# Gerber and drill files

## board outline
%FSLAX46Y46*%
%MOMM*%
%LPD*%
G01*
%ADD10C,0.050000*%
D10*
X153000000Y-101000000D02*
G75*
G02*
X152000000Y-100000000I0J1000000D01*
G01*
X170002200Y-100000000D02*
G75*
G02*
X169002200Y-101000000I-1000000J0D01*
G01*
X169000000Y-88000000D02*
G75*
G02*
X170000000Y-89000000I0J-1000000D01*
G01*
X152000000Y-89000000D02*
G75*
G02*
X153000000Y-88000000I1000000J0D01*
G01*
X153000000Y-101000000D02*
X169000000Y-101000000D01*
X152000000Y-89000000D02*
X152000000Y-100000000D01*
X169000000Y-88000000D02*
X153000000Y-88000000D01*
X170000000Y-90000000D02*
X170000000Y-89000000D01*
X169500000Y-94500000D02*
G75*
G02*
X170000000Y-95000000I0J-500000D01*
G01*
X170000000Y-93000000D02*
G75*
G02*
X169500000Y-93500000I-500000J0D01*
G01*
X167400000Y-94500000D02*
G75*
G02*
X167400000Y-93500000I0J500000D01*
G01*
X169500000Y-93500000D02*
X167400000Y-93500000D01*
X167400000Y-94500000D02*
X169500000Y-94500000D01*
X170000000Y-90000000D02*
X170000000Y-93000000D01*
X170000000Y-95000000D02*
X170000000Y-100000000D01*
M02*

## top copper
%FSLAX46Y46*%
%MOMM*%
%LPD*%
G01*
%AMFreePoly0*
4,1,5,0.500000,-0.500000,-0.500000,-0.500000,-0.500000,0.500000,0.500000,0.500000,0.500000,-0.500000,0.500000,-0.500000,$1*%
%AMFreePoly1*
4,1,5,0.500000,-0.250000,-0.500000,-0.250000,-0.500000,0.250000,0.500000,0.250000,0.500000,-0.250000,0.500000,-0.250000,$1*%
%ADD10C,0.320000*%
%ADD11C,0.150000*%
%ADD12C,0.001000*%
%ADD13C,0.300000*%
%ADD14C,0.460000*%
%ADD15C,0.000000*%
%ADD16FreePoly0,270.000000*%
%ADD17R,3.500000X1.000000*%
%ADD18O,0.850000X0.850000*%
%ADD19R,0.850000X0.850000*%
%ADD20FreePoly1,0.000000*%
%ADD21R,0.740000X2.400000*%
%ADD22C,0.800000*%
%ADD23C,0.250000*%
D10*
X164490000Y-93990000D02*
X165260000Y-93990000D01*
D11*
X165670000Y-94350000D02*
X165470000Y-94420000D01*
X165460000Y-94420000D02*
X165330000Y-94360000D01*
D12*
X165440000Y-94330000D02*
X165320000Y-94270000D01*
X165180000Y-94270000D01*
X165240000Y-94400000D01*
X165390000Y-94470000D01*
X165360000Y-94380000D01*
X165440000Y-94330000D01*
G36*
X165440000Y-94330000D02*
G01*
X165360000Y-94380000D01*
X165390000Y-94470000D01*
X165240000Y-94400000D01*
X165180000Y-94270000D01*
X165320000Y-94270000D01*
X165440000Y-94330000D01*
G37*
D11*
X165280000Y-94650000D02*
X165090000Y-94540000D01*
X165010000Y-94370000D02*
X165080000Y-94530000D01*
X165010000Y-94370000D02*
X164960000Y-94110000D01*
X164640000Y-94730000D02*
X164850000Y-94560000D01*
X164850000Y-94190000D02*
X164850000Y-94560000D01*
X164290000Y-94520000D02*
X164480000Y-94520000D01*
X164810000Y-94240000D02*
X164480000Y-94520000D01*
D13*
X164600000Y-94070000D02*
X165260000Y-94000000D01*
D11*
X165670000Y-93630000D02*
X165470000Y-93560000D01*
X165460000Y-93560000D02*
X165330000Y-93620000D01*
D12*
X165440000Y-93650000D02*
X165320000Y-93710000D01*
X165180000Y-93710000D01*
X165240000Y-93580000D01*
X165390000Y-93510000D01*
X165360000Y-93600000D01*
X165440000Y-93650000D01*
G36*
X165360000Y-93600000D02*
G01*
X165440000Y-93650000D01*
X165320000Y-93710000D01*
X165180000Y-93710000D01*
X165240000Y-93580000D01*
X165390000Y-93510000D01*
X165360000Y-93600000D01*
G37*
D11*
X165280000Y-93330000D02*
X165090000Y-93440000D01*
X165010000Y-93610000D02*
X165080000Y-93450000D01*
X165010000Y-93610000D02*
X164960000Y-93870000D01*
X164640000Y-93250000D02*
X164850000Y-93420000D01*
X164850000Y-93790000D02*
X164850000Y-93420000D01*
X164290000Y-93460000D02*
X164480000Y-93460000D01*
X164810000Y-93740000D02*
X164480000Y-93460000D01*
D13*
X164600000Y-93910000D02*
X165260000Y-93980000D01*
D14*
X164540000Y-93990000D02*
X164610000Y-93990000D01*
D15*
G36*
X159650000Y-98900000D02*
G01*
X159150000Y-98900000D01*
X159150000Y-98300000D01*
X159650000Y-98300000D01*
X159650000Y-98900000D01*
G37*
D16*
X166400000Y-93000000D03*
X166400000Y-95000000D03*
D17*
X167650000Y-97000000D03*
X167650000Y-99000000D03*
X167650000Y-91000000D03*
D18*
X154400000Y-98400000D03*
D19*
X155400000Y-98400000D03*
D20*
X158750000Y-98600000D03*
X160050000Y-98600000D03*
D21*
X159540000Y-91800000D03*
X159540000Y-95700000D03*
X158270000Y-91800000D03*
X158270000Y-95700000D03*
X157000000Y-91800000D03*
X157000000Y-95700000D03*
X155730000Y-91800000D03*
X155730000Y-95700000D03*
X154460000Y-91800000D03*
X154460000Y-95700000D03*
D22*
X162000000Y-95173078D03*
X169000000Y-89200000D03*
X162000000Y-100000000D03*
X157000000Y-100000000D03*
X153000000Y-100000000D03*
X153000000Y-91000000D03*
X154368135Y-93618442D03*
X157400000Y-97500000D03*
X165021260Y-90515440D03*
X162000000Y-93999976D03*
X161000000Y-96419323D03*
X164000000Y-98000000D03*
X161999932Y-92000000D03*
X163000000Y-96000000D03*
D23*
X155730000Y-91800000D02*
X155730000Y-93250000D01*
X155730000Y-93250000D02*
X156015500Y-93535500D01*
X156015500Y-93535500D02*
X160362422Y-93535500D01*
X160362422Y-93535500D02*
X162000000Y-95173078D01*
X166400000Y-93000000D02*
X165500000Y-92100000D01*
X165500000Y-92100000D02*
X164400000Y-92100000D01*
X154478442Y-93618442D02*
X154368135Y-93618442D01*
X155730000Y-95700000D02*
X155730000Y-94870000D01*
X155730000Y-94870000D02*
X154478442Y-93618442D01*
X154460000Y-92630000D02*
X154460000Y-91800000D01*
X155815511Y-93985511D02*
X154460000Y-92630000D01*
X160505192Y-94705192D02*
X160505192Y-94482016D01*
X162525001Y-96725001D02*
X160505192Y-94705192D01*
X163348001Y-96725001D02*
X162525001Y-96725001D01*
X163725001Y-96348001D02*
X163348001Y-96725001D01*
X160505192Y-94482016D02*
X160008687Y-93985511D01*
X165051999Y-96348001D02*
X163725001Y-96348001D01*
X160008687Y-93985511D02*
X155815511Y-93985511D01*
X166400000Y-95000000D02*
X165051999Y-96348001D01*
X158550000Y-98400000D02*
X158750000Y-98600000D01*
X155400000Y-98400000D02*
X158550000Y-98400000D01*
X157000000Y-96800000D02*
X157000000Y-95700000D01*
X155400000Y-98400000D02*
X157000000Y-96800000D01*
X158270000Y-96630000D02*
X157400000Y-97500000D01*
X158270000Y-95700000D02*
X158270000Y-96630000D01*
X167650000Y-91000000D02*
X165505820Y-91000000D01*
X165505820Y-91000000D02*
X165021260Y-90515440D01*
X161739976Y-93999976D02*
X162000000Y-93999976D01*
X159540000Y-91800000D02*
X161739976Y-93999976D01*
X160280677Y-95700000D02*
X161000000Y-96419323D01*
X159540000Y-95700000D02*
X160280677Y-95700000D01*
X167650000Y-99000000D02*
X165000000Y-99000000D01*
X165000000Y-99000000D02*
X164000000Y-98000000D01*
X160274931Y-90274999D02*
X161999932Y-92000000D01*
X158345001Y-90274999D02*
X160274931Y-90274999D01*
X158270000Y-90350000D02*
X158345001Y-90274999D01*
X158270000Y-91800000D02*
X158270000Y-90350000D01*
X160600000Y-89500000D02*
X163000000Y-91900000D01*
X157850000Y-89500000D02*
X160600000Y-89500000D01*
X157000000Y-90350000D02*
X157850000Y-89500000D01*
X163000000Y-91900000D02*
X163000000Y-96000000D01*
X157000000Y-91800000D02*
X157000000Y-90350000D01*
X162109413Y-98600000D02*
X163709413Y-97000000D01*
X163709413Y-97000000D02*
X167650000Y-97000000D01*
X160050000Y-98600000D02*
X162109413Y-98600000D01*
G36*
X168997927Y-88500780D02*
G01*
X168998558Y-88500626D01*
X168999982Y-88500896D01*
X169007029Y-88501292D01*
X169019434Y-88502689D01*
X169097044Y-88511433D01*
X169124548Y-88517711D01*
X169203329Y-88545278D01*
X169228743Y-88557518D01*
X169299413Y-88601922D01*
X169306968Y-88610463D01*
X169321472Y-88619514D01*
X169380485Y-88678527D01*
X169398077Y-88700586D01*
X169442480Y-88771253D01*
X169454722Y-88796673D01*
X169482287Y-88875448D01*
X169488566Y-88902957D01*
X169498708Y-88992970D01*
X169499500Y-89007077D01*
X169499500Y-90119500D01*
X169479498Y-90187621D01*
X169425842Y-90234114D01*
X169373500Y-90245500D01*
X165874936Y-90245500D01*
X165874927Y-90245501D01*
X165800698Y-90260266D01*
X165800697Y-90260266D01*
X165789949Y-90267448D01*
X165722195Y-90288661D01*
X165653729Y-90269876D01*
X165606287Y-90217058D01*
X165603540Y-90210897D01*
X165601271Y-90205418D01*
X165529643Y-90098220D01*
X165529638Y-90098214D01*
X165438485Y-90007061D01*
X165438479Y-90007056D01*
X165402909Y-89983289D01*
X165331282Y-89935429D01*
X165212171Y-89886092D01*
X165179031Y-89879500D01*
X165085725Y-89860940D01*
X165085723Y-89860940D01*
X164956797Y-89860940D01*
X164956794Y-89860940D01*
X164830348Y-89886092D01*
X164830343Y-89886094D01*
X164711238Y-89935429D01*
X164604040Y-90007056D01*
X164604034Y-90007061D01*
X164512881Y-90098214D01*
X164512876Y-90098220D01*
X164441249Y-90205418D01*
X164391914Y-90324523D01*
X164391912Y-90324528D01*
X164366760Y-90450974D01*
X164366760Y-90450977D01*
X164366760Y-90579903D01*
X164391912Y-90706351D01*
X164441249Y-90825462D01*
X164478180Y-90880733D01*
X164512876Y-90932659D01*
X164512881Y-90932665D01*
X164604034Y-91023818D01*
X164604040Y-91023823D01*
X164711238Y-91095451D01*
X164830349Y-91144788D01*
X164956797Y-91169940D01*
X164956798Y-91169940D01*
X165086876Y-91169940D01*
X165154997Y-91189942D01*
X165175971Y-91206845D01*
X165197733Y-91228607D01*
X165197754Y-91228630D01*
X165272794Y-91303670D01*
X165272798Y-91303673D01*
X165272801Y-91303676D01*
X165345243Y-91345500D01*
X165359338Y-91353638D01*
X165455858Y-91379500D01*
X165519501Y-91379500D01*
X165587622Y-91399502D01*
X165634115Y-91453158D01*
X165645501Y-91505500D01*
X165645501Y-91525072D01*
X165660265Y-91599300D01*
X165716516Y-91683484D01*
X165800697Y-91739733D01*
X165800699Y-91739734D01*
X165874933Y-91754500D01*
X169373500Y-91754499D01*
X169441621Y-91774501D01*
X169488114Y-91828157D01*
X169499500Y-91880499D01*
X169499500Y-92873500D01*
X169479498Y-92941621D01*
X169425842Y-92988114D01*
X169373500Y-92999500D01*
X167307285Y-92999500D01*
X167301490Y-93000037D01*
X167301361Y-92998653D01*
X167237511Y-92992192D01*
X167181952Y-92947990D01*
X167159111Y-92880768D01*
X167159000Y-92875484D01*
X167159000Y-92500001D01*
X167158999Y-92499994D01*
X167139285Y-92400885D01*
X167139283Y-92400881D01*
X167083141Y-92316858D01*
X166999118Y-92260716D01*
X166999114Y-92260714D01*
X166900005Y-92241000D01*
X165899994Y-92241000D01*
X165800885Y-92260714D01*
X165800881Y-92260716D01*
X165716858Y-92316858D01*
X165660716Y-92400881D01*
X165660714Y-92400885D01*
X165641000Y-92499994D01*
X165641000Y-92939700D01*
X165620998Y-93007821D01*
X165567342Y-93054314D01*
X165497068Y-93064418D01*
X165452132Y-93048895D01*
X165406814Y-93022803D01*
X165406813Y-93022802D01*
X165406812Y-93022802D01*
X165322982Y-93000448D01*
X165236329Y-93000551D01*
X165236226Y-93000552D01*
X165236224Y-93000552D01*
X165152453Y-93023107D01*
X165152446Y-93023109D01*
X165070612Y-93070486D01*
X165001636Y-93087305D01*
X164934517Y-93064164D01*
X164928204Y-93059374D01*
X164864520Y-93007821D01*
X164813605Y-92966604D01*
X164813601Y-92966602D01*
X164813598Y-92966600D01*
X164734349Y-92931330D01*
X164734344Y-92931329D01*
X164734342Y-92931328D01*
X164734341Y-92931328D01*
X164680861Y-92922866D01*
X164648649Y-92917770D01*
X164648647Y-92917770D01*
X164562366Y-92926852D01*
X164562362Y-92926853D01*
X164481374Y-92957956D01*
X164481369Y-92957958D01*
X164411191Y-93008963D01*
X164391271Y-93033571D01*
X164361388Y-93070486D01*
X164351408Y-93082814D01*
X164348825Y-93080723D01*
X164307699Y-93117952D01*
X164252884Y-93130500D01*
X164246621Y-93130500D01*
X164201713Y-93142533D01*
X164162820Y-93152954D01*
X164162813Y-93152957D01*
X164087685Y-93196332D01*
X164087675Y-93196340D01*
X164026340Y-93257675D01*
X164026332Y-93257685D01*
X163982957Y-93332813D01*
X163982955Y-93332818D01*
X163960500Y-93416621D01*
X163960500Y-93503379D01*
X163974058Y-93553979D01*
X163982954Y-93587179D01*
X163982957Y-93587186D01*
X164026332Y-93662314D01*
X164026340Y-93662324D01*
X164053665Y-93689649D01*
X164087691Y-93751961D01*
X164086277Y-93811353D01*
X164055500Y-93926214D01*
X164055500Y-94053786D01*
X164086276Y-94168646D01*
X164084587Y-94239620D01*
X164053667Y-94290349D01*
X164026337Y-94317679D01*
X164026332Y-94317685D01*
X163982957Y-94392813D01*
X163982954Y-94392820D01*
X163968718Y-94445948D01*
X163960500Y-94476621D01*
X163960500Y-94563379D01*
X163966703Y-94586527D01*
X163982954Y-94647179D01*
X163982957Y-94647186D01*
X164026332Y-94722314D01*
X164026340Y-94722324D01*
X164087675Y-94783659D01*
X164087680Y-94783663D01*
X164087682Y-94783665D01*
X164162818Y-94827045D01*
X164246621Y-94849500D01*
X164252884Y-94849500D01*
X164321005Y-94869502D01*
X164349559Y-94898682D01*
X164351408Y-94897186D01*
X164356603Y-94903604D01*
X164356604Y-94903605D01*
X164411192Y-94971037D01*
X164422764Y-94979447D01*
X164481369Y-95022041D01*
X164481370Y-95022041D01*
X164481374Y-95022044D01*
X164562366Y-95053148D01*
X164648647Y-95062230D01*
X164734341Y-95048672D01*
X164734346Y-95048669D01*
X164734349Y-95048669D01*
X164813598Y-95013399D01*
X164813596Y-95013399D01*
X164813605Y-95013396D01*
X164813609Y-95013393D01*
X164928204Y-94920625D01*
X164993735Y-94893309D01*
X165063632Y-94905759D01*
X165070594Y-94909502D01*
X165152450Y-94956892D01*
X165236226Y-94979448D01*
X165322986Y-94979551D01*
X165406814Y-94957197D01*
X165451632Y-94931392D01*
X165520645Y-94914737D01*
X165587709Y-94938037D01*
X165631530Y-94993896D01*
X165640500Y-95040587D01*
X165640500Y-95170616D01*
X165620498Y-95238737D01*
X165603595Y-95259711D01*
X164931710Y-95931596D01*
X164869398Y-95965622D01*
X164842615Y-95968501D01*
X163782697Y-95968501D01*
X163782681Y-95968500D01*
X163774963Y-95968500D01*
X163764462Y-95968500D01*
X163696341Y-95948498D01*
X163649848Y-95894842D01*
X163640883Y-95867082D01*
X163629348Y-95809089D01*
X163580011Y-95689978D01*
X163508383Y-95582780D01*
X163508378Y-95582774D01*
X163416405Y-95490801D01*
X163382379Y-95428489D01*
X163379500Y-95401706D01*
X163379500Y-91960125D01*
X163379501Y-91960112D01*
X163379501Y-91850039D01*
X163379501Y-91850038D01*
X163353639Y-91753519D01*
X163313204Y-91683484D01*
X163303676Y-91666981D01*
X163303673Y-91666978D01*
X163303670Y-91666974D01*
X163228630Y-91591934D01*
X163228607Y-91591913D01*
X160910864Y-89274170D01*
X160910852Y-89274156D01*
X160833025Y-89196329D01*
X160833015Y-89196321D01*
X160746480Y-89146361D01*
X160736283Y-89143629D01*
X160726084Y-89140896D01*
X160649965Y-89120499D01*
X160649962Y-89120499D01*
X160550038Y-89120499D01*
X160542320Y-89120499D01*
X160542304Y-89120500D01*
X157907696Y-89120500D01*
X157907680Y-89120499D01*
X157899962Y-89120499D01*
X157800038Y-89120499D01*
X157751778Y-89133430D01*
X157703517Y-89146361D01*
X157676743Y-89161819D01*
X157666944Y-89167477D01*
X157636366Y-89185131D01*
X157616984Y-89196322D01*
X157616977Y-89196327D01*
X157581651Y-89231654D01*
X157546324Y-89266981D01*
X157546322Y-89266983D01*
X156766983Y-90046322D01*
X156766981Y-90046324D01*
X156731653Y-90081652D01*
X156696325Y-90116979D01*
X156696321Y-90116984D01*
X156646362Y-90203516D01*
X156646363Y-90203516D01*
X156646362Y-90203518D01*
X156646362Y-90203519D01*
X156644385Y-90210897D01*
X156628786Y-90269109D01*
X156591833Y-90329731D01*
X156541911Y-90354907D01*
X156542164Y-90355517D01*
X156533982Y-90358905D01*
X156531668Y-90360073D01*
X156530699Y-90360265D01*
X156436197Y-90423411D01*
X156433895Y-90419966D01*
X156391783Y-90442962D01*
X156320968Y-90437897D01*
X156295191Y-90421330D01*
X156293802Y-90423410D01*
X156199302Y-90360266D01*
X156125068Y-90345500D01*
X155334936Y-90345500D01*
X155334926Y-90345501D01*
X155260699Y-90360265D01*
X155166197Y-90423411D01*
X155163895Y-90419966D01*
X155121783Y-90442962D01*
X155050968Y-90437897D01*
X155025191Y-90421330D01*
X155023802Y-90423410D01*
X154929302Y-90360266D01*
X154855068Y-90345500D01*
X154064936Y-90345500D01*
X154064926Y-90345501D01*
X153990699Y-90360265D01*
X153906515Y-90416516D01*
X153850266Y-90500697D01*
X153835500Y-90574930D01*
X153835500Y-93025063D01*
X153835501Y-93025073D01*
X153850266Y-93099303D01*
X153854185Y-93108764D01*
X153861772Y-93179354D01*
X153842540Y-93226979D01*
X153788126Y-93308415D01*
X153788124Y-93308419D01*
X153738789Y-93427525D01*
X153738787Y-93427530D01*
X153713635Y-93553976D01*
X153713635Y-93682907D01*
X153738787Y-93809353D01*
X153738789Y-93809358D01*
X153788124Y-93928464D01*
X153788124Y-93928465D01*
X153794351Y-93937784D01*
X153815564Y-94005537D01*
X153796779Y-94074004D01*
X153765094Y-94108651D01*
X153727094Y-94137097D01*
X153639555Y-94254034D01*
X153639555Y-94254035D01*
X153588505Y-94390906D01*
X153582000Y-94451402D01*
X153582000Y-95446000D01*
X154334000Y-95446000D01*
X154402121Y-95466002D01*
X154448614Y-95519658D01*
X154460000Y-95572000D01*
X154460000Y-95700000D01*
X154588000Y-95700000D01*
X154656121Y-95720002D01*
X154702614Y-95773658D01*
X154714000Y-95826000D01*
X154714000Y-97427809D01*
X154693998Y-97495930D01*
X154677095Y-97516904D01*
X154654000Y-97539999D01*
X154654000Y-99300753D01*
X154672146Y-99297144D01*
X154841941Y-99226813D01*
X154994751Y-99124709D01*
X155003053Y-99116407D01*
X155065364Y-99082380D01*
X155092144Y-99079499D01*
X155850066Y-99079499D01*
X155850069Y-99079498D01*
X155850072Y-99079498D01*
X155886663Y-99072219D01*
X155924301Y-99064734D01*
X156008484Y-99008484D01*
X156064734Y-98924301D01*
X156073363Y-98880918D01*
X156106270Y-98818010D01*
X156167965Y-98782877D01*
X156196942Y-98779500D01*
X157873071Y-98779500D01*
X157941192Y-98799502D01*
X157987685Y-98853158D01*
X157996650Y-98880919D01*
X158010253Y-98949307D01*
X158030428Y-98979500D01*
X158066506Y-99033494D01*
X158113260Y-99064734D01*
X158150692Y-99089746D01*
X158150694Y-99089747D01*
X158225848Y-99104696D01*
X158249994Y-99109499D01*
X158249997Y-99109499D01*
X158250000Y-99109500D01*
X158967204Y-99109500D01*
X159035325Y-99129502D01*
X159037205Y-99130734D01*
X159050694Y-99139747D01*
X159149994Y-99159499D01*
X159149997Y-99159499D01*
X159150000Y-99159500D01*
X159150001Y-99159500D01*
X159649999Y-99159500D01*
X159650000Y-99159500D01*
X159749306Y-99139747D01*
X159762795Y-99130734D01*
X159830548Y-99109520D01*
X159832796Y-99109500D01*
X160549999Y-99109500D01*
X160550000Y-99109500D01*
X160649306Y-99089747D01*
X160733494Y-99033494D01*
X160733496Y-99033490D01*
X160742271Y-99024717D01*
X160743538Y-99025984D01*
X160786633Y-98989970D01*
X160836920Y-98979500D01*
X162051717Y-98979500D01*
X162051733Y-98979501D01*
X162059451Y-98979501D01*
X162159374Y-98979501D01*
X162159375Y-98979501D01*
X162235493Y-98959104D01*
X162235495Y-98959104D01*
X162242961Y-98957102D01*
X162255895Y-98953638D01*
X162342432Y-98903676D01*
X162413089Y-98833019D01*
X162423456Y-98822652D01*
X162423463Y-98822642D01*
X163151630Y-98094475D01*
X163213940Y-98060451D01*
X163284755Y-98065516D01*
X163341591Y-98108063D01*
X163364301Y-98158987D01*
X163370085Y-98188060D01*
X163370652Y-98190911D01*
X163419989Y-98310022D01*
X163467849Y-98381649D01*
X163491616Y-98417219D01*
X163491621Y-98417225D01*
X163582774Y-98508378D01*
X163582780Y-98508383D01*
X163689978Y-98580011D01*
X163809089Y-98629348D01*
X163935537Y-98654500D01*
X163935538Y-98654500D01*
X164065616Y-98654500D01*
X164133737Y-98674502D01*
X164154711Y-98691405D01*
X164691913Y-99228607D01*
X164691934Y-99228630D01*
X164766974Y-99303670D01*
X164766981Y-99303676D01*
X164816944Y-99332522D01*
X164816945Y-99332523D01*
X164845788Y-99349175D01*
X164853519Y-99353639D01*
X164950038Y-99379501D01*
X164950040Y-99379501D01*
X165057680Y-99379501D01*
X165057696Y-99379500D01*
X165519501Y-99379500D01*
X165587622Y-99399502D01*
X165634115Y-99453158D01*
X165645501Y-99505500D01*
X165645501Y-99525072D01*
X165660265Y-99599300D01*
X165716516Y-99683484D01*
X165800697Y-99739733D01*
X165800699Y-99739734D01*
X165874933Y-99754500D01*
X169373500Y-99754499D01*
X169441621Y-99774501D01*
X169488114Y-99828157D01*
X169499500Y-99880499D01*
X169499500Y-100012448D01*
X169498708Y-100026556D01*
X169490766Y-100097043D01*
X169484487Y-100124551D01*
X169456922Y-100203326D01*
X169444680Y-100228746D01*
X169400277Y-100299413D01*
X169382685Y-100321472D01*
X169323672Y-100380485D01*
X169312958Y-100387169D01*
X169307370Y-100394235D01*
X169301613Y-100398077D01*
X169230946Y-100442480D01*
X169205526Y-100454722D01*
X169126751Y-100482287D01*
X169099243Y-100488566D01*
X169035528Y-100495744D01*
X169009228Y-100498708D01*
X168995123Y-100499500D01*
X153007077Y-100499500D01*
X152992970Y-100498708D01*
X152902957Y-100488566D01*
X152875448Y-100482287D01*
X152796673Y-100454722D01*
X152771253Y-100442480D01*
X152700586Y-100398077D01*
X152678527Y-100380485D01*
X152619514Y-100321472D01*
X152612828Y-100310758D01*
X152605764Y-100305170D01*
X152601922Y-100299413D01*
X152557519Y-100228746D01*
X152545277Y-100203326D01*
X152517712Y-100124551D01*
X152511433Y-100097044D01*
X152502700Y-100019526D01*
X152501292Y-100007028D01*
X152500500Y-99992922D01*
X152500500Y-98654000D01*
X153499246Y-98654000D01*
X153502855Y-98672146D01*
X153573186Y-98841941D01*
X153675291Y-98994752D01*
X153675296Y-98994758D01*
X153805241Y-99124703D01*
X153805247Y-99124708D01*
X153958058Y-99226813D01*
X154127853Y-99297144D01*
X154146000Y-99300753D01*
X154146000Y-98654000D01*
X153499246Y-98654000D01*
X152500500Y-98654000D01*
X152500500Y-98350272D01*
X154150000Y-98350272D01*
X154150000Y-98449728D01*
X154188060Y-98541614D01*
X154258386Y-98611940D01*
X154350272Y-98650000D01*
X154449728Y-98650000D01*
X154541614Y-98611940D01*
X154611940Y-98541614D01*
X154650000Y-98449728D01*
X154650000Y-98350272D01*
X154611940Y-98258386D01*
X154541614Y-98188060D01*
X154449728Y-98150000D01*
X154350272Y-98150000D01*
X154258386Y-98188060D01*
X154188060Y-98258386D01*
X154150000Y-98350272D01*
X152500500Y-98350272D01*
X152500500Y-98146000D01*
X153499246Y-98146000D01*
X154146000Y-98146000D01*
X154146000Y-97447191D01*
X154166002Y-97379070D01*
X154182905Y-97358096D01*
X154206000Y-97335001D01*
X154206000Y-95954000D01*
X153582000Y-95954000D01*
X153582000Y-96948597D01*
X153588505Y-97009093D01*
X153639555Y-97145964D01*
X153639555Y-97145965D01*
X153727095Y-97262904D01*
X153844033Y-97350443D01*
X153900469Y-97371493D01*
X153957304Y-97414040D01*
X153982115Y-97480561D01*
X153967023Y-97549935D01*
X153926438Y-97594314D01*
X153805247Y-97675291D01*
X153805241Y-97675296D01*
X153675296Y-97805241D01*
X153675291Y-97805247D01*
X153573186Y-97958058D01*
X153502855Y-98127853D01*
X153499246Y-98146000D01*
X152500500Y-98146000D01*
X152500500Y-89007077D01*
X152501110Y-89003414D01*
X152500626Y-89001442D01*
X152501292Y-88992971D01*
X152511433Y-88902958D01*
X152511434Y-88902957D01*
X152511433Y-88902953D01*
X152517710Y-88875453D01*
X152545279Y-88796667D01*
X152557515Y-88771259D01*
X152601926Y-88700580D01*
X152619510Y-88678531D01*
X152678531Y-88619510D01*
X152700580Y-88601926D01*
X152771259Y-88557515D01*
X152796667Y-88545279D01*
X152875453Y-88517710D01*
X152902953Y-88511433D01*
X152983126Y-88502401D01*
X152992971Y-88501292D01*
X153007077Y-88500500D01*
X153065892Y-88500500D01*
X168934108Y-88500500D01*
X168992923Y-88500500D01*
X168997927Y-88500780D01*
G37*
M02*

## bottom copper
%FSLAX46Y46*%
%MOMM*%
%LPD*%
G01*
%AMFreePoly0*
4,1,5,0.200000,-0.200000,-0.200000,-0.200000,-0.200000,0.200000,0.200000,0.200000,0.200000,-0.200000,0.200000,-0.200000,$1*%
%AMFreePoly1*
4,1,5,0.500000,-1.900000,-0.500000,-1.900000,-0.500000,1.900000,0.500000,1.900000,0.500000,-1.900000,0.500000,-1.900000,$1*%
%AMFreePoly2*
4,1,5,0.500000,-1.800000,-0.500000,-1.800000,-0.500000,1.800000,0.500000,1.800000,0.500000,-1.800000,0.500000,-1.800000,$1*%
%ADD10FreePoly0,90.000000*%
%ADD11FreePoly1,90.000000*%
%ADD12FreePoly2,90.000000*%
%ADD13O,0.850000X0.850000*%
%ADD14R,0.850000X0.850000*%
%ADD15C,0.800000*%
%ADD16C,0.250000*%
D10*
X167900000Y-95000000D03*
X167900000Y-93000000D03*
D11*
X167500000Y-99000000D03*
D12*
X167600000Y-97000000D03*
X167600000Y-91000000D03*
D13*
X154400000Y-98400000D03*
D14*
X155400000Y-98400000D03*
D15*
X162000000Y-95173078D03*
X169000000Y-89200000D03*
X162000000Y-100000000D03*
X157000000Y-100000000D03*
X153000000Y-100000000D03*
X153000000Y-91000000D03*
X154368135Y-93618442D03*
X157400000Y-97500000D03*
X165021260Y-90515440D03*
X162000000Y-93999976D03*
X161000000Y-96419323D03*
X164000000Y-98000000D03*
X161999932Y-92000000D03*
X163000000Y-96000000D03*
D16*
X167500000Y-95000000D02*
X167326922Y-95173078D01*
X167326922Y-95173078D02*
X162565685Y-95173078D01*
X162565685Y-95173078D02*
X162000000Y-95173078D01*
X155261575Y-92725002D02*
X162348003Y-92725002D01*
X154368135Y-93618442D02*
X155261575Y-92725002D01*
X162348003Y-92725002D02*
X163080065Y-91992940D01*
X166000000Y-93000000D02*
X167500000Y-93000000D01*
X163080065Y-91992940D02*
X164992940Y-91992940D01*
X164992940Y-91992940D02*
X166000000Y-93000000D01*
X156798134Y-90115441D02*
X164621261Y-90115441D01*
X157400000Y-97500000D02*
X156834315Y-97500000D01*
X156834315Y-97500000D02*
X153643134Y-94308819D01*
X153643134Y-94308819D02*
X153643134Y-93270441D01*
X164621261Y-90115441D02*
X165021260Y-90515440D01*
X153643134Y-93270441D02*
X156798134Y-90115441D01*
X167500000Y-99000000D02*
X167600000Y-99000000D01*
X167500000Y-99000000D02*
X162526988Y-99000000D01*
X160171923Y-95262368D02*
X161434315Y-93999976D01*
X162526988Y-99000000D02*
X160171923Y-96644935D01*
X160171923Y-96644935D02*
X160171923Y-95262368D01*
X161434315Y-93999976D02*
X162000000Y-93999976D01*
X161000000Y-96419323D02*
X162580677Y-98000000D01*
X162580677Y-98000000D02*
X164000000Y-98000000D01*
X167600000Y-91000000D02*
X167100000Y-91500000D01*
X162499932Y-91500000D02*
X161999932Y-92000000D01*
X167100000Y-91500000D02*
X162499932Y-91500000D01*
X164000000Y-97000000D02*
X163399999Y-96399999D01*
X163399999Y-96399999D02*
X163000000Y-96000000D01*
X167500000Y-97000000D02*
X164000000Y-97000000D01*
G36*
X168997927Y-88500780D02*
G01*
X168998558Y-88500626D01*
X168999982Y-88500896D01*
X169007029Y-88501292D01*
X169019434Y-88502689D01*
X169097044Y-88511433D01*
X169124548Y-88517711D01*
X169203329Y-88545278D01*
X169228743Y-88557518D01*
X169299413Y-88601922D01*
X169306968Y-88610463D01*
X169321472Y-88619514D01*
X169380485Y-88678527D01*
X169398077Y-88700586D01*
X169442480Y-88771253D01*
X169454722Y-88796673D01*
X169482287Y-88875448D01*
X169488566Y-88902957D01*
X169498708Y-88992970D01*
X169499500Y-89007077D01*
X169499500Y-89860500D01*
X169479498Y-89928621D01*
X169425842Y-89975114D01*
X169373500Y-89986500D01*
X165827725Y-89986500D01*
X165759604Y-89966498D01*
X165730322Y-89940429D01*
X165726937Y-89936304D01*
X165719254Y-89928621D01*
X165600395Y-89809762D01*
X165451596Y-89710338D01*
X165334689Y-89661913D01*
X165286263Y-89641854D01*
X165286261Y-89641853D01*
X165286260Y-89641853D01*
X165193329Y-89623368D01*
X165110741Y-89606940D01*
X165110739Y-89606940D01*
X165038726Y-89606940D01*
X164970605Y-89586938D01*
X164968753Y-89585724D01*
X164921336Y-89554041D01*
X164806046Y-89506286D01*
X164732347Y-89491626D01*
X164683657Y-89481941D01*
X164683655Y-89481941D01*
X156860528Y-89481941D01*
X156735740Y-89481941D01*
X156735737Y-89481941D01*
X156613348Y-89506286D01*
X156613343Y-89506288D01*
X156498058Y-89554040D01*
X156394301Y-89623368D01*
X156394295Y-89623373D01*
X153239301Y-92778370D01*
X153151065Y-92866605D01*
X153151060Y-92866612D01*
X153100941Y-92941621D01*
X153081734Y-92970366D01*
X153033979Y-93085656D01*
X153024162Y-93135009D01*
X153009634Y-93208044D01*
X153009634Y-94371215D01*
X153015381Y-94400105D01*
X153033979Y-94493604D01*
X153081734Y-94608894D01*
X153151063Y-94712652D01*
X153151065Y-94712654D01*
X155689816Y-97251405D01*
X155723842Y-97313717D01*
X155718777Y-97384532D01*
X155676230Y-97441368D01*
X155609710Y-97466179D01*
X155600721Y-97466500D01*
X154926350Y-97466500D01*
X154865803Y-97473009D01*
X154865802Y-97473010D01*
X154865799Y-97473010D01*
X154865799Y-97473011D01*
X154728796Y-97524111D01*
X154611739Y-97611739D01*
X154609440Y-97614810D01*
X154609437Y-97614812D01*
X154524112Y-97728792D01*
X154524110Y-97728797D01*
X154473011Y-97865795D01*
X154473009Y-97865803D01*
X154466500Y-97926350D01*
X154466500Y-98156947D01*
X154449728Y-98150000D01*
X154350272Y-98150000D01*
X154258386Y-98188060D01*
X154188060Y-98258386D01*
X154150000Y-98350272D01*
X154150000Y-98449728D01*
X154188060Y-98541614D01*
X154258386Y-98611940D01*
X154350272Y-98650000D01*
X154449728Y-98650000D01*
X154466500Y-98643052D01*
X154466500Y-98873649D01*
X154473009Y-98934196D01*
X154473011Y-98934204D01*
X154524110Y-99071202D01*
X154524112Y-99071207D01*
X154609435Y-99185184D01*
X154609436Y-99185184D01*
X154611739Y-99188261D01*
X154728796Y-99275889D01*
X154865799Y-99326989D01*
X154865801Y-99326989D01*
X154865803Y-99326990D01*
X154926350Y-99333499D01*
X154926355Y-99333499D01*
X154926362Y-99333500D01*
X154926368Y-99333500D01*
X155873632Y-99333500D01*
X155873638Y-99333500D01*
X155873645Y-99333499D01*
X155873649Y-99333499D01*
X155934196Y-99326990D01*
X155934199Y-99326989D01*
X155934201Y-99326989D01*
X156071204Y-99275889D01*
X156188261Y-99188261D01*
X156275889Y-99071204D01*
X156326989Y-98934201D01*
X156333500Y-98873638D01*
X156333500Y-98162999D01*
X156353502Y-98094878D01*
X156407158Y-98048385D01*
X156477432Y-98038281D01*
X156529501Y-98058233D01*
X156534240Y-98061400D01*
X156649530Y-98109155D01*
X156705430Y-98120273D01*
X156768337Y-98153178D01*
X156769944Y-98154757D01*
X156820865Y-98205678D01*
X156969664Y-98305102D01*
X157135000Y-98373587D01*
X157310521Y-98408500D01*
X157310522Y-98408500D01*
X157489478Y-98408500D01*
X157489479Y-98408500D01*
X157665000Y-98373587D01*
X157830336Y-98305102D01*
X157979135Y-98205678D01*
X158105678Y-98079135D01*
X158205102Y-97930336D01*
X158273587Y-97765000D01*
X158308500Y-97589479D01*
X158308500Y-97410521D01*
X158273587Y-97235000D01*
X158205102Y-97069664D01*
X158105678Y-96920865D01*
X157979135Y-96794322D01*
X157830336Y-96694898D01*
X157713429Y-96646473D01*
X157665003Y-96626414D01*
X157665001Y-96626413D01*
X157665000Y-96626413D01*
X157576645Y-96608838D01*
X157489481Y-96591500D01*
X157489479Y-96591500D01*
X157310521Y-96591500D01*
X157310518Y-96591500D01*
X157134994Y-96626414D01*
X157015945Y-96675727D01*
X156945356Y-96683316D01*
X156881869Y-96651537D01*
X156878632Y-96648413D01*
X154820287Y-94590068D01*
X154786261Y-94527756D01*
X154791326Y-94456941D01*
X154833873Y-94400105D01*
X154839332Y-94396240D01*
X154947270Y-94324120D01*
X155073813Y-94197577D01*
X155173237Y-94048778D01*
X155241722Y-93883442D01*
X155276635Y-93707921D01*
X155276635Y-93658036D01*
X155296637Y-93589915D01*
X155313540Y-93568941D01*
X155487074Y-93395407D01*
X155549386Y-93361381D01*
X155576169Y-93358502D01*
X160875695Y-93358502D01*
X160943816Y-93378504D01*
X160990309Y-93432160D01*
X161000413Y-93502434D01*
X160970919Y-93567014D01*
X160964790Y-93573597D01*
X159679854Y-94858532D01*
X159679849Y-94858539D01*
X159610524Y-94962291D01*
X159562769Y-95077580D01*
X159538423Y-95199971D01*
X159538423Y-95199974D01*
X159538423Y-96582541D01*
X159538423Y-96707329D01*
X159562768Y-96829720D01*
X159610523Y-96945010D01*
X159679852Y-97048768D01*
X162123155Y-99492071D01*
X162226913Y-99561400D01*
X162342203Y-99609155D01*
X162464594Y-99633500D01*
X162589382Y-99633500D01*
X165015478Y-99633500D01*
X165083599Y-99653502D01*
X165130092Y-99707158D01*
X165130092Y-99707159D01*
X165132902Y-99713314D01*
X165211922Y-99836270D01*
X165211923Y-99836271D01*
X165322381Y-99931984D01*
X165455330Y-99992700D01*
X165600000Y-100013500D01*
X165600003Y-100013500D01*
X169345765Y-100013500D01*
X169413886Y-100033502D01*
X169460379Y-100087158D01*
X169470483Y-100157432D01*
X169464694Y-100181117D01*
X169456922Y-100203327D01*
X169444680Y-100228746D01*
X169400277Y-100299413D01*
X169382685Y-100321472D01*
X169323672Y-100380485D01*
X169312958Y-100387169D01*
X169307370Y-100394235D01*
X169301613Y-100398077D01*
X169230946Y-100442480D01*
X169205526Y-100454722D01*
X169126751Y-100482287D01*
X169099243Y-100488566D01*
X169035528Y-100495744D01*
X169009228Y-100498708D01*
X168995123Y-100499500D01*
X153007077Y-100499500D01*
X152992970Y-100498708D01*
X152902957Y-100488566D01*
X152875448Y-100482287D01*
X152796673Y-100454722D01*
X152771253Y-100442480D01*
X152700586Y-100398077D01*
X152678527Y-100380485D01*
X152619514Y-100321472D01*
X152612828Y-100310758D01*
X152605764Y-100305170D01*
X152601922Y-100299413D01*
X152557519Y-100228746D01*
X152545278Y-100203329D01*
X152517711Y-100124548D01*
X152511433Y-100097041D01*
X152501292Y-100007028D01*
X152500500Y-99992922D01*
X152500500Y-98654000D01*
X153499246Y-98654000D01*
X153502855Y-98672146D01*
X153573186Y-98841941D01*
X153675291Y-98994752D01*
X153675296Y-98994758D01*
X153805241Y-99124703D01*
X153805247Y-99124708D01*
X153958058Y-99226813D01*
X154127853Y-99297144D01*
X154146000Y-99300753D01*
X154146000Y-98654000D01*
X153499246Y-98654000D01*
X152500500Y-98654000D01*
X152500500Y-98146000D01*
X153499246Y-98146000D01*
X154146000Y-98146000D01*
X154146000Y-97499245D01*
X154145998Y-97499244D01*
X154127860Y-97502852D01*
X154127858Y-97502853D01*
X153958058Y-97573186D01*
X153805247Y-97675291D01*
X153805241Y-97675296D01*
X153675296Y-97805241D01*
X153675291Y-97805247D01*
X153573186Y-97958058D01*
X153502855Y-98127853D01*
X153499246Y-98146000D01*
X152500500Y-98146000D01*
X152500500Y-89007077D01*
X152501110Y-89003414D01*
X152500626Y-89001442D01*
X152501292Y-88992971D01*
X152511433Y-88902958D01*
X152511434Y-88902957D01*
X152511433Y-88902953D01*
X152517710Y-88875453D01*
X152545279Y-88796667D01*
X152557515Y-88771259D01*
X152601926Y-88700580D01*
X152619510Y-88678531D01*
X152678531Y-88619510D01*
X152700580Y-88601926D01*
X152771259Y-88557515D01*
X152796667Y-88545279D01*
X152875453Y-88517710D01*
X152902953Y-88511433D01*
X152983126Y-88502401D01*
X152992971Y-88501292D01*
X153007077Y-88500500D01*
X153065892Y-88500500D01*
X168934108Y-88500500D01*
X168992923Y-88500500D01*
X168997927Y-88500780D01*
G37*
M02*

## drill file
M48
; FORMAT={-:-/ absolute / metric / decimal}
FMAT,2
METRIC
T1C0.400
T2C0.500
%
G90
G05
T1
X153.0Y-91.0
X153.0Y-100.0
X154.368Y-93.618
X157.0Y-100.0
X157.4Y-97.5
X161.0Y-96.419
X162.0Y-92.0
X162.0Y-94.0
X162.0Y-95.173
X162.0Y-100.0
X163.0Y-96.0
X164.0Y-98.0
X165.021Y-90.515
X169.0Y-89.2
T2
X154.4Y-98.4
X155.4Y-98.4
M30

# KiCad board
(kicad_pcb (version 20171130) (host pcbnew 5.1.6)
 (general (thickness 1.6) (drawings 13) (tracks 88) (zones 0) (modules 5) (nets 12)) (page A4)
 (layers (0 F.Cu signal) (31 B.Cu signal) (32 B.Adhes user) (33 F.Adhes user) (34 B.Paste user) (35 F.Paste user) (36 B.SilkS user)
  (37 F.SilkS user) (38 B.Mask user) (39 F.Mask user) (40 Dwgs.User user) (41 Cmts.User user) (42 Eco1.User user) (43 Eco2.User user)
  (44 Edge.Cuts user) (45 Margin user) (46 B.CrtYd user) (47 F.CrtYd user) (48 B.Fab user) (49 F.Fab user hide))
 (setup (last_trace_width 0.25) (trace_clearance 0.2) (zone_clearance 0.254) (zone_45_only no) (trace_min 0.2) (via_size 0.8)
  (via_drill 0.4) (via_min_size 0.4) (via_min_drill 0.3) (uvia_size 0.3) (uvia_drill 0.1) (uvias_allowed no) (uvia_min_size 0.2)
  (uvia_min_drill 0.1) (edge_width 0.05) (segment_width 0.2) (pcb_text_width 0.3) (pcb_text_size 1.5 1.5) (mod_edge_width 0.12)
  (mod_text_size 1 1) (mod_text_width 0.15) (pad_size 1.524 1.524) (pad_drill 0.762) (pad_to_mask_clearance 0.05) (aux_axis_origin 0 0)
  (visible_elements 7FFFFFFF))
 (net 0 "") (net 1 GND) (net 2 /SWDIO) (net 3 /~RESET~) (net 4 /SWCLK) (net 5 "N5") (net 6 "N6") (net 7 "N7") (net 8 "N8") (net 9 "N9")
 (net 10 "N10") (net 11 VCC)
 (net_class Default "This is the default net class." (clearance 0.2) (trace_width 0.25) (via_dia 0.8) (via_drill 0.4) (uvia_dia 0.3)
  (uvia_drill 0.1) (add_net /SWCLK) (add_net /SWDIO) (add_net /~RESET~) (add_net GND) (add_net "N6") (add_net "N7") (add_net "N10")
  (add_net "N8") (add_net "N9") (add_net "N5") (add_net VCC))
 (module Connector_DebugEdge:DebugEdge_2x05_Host (layer F.Cu) (at 170 95 270)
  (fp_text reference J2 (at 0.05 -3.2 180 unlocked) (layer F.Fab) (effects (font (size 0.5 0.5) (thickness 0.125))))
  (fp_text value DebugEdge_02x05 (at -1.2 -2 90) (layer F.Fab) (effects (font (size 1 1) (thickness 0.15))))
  (fp_arc (start 0 0.5) (end 0 0) (angle -90) (layer Edge.Cuts) (width 0.05))
  (fp_arc (start -2 0.5) (end -1.5 0.5) (angle -90) (layer Edge.Cuts) (width 0.05))
  (fp_arc (start -1 2.6) (end -1.5 2.6) (angle -180) (layer Edge.Cuts) (width 0.05))
  (fp_line (start -1.01 5.51) (end -1.01 4.74) (layer F.Cu) (width 0.32))
  (fp_line (start -0.65 4.33) (end -0.58 4.53) (layer F.Cu) (width 0.15))
  (fp_line (start -0.58 4.54) (end -0.64 4.67) (layer F.Cu) (width 0.15))
  (fp_poly (pts (xy -0.67 4.56) (xy -0.73 4.68) (xy -0.73 4.82) (xy -0.6 4.76) (xy -0.53 4.61) (xy -0.62 4.64)) (layer F.Cu) (width 0.001))
  (fp_line (start -0.35 4.72) (end -0.46 4.91) (layer F.Cu) (width 0.15))
  (fp_line (start -0.63 4.99) (end -0.47 4.92) (layer F.Cu) (width 0.15))
  (fp_line (start -0.63 4.99) (end -0.89 5.04) (layer F.Cu) (width 0.15))
  (fp_line (start -0.27 5.36) (end -0.44 5.15) (layer F.Cu) (width 0.15))
  (fp_line (start -0.81 5.15) (end -0.44 5.15) (layer F.Cu) (width 0.15))
  (fp_line (start -0.48 5.71) (end -0.48 5.52) (layer F.Cu) (width 0.15))
  (fp_line (start -0.76 5.19) (end -0.48 5.52) (layer F.Cu) (width 0.15))
  (fp_line (start -0.93 5.4) (end -1 4.74) (layer F.Cu) (width 0.3))
  (fp_line (start -1.5 0.5) (end -1.5 2.6) (layer Edge.Cuts) (width 0.05))
  (fp_line (start -0.5 2.6) (end -0.5 0.5) (layer Edge.Cuts) (width 0.05))
  (fp_line (start -5 0) (end -2 0) (layer Edge.Cuts) (width 0.05))
  (fp_line (start 0 0) (end 5 0) (layer Edge.Cuts) (width 0.05))
  (fp_line (start -1.37 4.33) (end -1.44 4.53) (layer F.Cu) (width 0.15))
  (fp_line (start -1.44 4.54) (end -1.38 4.67) (layer F.Cu) (width 0.15))
  (fp_poly (pts (xy -1.35 4.56) (xy -1.29 4.68) (xy -1.29 4.82) (xy -1.42 4.76) (xy -1.49 4.61) (xy -1.4 4.64)) (layer F.Cu) (width 0.001))
  (fp_line (start -1.67 4.72) (end -1.56 4.91) (layer F.Cu) (width 0.15))
  (fp_line (start -1.39 4.99) (end -1.55 4.92) (layer F.Cu) (width 0.15))
  (fp_line (start -1.39 4.99) (end -1.13 5.04) (layer F.Cu) (width 0.15))
  (fp_line (start -1.75 5.36) (end -1.58 5.15) (layer F.Cu) (width 0.15))
  (fp_line (start -1.21 5.15) (end -1.58 5.15) (layer F.Cu) (width 0.15))
  (fp_line (start -1.54 5.71) (end -1.54 5.52) (layer F.Cu) (width 0.15))
  (fp_line (start -1.26 5.19) (end -1.54 5.52) (layer F.Cu) (width 0.15))
  (fp_line (start -1.09 5.4) (end -1.02 4.74) (layer F.Cu) (width 0.3))
  (fp_line (start -1.01 5.46) (end -1.01 5.39) (layer F.Cu) (width 0.46))
  (pad 1 smd custom (at -2 3.6 270) (size 1 1) (layers F.Cu F.Mask) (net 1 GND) (zone_connect 0) (options (clearance outline) (anchor rect))
   (primitives))
  (pad 2 smd custom (at 0 3.6 270) (size 1 1) (layers F.Cu F.Mask) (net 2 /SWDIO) (zone_connect 0)
   (options (clearance outline) (anchor rect)) (primitives))
  (pad 4 smd custom (at 0 2.1 90) (size 0.4 0.4) (layers B.Cu B.Mask) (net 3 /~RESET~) (zone_connect 0)
   (options (clearance outline) (anchor rect)) (primitives))
  (pad 3 smd custom (at -2 2.1 90) (size 0.4 0.4) (layers B.Cu B.Mask) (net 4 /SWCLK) (zone_connect 0)
   (options (clearance outline) (anchor rect)) (primitives))
  (pad 5 smd rect (at 2 2.35 270) (size 1 3.5) (layers F.Cu F.Mask) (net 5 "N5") (zone_connect 0))
  (pad 10 smd custom (at 4 2.5 90) (size 1 3.8) (layers B.Cu B.Mask) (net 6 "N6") (zone_connect 0)
   (options (clearance outline) (anchor rect)) (primitives))
  (pad 6 smd custom (at 2 2.4 90) (size 1 3.6) (layers B.Cu B.Mask) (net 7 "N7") (zone_connect 0)
   (options (clearance outline) (anchor rect)) (primitives))
  (pad 8 smd custom (at -4 2.4 90) (size 1 3.6) (layers B.Cu B.Mask) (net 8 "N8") (zone_connect 0)
   (options (clearance outline) (anchor rect)) (primitives))
  (pad 9 smd rect (at 4 2.35 270) (size 1 3.5) (layers F.Cu F.Mask) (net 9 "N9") (zone_connect 0))
  (pad 7 smd rect (at -4 2.35 270) (size 1 3.5) (layers F.Cu F.Mask) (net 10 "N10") (zone_connect 0)))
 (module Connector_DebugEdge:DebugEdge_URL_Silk (layer F.Cu) (at 161.6 89 180)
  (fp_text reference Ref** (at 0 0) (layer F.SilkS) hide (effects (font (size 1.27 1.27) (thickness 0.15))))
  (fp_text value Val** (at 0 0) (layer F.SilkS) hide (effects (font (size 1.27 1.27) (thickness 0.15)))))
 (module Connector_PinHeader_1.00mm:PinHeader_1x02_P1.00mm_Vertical (layer F.Cu) (at 155.4 98.4 270)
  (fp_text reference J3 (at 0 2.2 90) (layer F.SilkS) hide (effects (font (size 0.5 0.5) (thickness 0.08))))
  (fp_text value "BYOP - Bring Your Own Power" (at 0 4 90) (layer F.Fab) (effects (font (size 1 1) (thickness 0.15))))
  (pad 2 thru_hole oval (at 0 1 270) (size 0.85 0.85) (drill 0.5) (layers *.Cu *.Mask) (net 1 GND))
  (pad 1 thru_hole rect (at 0 0 270) (size 0.85 0.85) (drill 0.5) (layers *.Cu *.Mask) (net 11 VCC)))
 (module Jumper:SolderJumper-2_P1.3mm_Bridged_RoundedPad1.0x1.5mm (layer F.Cu) (at 159.4 98.6)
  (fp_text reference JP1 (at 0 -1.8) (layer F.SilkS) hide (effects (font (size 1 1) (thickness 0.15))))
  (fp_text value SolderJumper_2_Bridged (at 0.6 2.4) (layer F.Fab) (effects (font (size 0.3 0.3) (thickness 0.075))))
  (fp_poly (pts (xy 0.25 -0.3) (xy -0.25 -0.3) (xy -0.25 0.3) (xy 0.25 0.3)) (layer F.Cu) (width 0))
  (pad 1 smd custom (at -0.65 0) (size 1 0.5) (layers F.Cu F.Mask) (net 11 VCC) (zone_connect 2) (options (clearance outline) (anchor rect))
   (primitives))
  (pad 2 smd custom (at 0.65 0) (size 1 0.5) (layers F.Cu F.Mask) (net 5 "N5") (zone_connect 2) (options (clearance outline) (anchor rect))
   (primitives)))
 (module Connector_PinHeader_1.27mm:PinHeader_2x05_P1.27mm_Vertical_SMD (layer F.Cu) (at 157 93.75 90)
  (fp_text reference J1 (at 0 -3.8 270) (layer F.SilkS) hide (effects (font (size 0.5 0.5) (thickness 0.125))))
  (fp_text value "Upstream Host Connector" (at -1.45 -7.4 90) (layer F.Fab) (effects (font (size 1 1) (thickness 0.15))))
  (pad 10 smd rect (at 1.95 2.54 90) (size 2.4 0.74) (layers F.Cu F.Paste F.Mask) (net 6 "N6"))
  (pad 9 smd rect (at -1.95 2.54 90) (size 2.4 0.74) (layers F.Cu F.Paste F.Mask) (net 9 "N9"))
  (pad 8 smd rect (at 1.95 1.27 90) (size 2.4 0.74) (layers F.Cu F.Paste F.Mask) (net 8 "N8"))
  (pad 7 smd rect (at -1.95 1.27 90) (size 2.4 0.74) (layers F.Cu F.Paste F.Mask) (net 10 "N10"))
  (pad 6 smd rect (at 1.95 0 90) (size 2.4 0.74) (layers F.Cu F.Paste F.Mask) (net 7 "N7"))
  (pad 5 smd rect (at -1.95 0 90) (size 2.4 0.74) (layers F.Cu F.Paste F.Mask) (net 11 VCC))
  (pad 4 smd rect (at 1.95 -1.27 90) (size 2.4 0.74) (layers F.Cu F.Paste F.Mask) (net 3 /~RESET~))
  (pad 3 smd rect (at -1.95 -1.27 90) (size 2.4 0.74) (layers F.Cu F.Paste F.Mask) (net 4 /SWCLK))
  (pad 2 smd rect (at 1.95 -2.54 90) (size 2.4 0.74) (layers F.Cu F.Paste F.Mask) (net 2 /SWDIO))
  (pad 1 smd rect (at -1.95 -2.54 90) (size 2.4 0.74) (layers F.Cu F.Paste F.Mask) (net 1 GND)))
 (gr_arc (start 153 100) (end 152 100) (angle -90) (layer Edge.Cuts) (width 0.05))
 (gr_arc (start 169.0022 100) (end 169.0022 101) (angle -90) (layer Edge.Cuts) (width 0.05))
 (gr_arc (start 169 89) (end 170 89) (angle -90) (layer Edge.Cuts) (width 0.05))
 (gr_arc (start 153 89) (end 153 88) (angle -90) (layer Edge.Cuts) (width 0.05))
 (gr_line (start 153 101) (end 169 101) (layer Edge.Cuts) (width 0.05))
 (gr_line (start 152 89) (end 152 100) (layer Edge.Cuts) (width 0.05))
 (gr_line (start 169 88) (end 153 88) (layer Edge.Cuts) (width 0.05))
 (gr_line (start 170 90) (end 170 89) (layer Edge.Cuts) (width 0.05))
 (via (at 162 95.173078) (size 0.8) (drill 0.4) (layers F.Cu B.Cu) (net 3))
 (segment (start 155.73 91.8) (end 155.73 93.25) (width 0.25) (layer F.Cu) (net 3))
 (segment (start 155.73 93.25) (end 156.0155 93.5355) (width 0.25) (layer F.Cu) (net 3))
 (segment (start 167.5 95) (end 167.326922 95.173078) (width 0.25) (layer B.Cu) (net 3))
 (segment (start 156.0155 93.5355) (end 160.362422 93.5355) (width 0.25) (layer F.Cu) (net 3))
 (segment (start 160.362422 93.5355) (end 162 95.173078) (width 0.25) (layer F.Cu) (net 3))
 (segment (start 167.326922 95.173078) (end 162.565685 95.173078) (width 0.25) (layer B.Cu) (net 3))
 (segment (start 162.565685 95.173078) (end 162 95.173078) (width 0.25) (layer B.Cu) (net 3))
 (via (at 169 89.2) (size 0.8) (drill 0.4) (layers F.Cu B.Cu) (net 1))
 (via (at 162 100) (size 0.8) (drill 0.4) (layers F.Cu B.Cu) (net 1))
 (via (at 157 100) (size 0.8) (drill 0.4) (layers F.Cu B.Cu) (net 1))
 (via (at 153 100) (size 0.8) (drill 0.4) (layers F.Cu B.Cu) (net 1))
 (via (at 153 91) (size 0.8) (drill 0.4) (layers F.Cu B.Cu) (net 1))
 (segment (start 166.4 93) (end 165.5 92.1) (width 0.25) (layer F.Cu) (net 1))
 (segment (start 165.5 92.1) (end 164.4 92.1) (width 0.25) (layer F.Cu) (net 1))
 (via (at 154.368135 93.618442) (size 0.8) (drill 0.4) (layers F.Cu B.Cu) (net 4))
 (segment (start 154.478442 93.618442) (end 154.368135 93.618442) (width 0.25) (layer F.Cu) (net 4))
 (segment (start 155.73 95.7) (end 155.73 94.87) (width 0.25) (layer F.Cu) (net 4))
 (segment (start 155.73 94.87) (end 154.478442 93.618442) (width 0.25) (layer F.Cu) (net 4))
 (segment (start 155.261575 92.725002) (end 162.348003 92.725002) (width 0.25) (layer B.Cu) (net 4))
 (segment (start 154.368135 93.618442) (end 155.261575 92.725002) (width 0.25) (layer B.Cu) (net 4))
 (segment (start 162.348003 92.725002) (end 163.080065 91.99294) (width 0.25) (layer B.Cu) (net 4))
 (segment (start 166 93) (end 167.5 93) (width 0.25) (layer B.Cu) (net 4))
 (segment (start 163.080065 91.99294) (end 164.99294 91.99294) (width 0.25) (layer B.Cu) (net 4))
 (segment (start 164.99294 91.99294) (end 166 93) (width 0.25) (layer B.Cu) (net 4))
 (segment (start 154.46 92.63) (end 154.46 91.8) (width 0.25) (layer F.Cu) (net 2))
 (segment (start 155.815511 93.985511) (end 154.46 92.63) (width 0.25) (layer F.Cu) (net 2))
 (segment (start 160.505192 94.705192) (end 160.505192 94.482016) (width 0.25) (layer F.Cu) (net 2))
 (segment (start 162.525001 96.725001) (end 160.505192 94.705192) (width 0.25) (layer F.Cu) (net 2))
 (segment (start 163.348001 96.725001) (end 162.525001 96.725001) (width 0.25) (layer F.Cu) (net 2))
 (segment (start 163.725001 96.348001) (end 163.348001 96.725001) (width 0.25) (layer F.Cu) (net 2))
 (segment (start 160.505192 94.482016) (end 160.008687 93.985511) (width 0.25) (layer F.Cu) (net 2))
 (segment (start 165.051999 96.348001) (end 163.725001 96.348001) (width 0.25) (layer F.Cu) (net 2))
 (segment (start 160.008687 93.985511) (end 155.815511 93.985511) (width 0.25) (layer F.Cu) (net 2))
 (segment (start 166.4 95) (end 165.051999 96.348001) (width 0.25) (layer F.Cu) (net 2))
 (segment (start 158.55 98.4) (end 158.75 98.6) (width 0.25) (layer F.Cu) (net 11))
 (segment (start 155.4 98.4) (end 158.55 98.4) (width 0.25) (layer F.Cu) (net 11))
 (segment (start 157 96.8) (end 157 95.7) (width 0.25) (layer F.Cu) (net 11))
 (segment (start 155.4 98.4) (end 157 96.8) (width 0.25) (layer F.Cu) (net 11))
 (segment (start 158.27 96.63) (end 157.4 97.5) (width 0.25) (layer F.Cu) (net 10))
 (via (at 157.4 97.5) (size 0.8) (drill 0.4) (layers F.Cu B.Cu) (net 10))
 (segment (start 158.27 95.7) (end 158.27 96.63) (width 0.25) (layer F.Cu) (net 10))
 (segment (start 156.798134 90.115441) (end 164.621261 90.115441) (width 0.25) (layer B.Cu) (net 10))
 (via (at 165.02126 90.51544) (size 0.8) (drill 0.4) (layers F.Cu B.Cu) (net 10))
 (segment (start 157.4 97.5) (end 156.834315 97.5) (width 0.25) (layer B.Cu) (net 10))
 (segment (start 156.834315 97.5) (end 153.643134 94.308819) (width 0.25) (layer B.Cu) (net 10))
 (segment (start 153.643134 94.308819) (end 153.643134 93.270441) (width 0.25) (layer B.Cu) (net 10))
 (segment (start 164.621261 90.115441) (end 165.02126 90.51544) (width 0.25) (layer B.Cu) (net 10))
 (segment (start 167.65 91) (end 165.50582 91) (width 0.25) (layer F.Cu) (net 10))
 (segment (start 153.643134 93.270441) (end 156.798134 90.115441) (width 0.25) (layer B.Cu) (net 10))
 (segment (start 165.50582 91) (end 165.02126 90.51544) (width 0.25) (layer F.Cu) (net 10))
 (segment (start 167.5 99) (end 167.6 99) (width 0.25) (layer B.Cu) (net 6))
 (via (at 162 93.999976) (size 0.8) (drill 0.4) (layers F.Cu B.Cu) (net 6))
 (segment (start 161.739976 93.999976) (end 162 93.999976) (width 0.25) (layer F.Cu) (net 6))
 (segment (start 159.54 91.8) (end 161.739976 93.999976) (width 0.25) (layer F.Cu) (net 6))
 (segment (start 167.5 99) (end 162.526988 99) (width 0.25) (layer B.Cu) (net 6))
 (segment (start 160.171923 95.262368) (end 161.434315 93.999976) (width 0.25) (layer B.Cu) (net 6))
 (segment (start 162.526988 99) (end 160.171923 96.644935) (width 0.25) (layer B.Cu) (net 6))
 (segment (start 160.171923 96.644935) (end 160.171923 95.262368) (width 0.25) (layer B.Cu) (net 6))
 (segment (start 161.434315 93.999976) (end 162 93.999976) (width 0.25) (layer B.Cu) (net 6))
 (segment (start 160.280677 95.7) (end 161 96.419323) (width 0.25) (layer F.Cu) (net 9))
 (segment (start 159.54 95.7) (end 160.280677 95.7) (width 0.25) (layer F.Cu) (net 9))
 (via (at 161 96.419323) (size 0.8) (drill 0.4) (layers F.Cu B.Cu) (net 9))
 (via (at 164 98) (size 0.8) (drill 0.4) (layers F.Cu B.Cu) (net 9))
 (segment (start 167.65 99) (end 165 99) (width 0.25) (layer F.Cu) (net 9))
 (segment (start 165 99) (end 164 98) (width 0.25) (layer F.Cu) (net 9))
 (segment (start 161 96.419323) (end 162.580677 98) (width 0.25) (layer B.Cu) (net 9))
 (segment (start 162.580677 98) (end 164 98) (width 0.25) (layer B.Cu) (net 9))
 (via (at 161.999932 92) (size 0.8) (drill 0.4) (layers F.Cu B.Cu) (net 8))
 (segment (start 167.6 91) (end 167.1 91.5) (width 0.25) (layer B.Cu) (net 8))
 (segment (start 160.274931 90.274999) (end 161.999932 92) (width 0.25) (layer F.Cu) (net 8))
 (segment (start 158.345001 90.274999) (end 160.274931 90.274999) (width 0.25) (layer F.Cu) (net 8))
 (segment (start 158.27 90.35) (end 158.345001 90.274999) (width 0.25) (layer F.Cu) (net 8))
 (segment (start 158.27 91.8) (end 158.27 90.35) (width 0.25) (layer F.Cu) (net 8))
 (segment (start 162.499932 91.5) (end 161.999932 92) (width 0.25) (layer B.Cu) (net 8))
 (segment (start 167.1 91.5) (end 162.499932 91.5) (width 0.25) (layer B.Cu) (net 8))
 (via (at 163 96) (size 0.8) (drill 0.4) (layers F.Cu B.Cu) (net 7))
 (segment (start 164 97) (end 163.399999 96.399999) (width 0.25) (layer B.Cu) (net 7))
 (segment (start 163.399999 96.399999) (end 163 96) (width 0.25) (layer B.Cu) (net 7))
 (segment (start 167.5 97) (end 164 97) (width 0.25) (layer B.Cu) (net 7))
 (segment (start 160.6 89.5) (end 163 91.9) (width 0.25) (layer F.Cu) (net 7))
 (segment (start 157.85 89.5) (end 160.6 89.5) (width 0.25) (layer F.Cu) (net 7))
 (segment (start 157 90.35) (end 157.85 89.5) (width 0.25) (layer F.Cu) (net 7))
 (segment (start 163 91.9) (end 163 96) (width 0.25) (layer F.Cu) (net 7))
 (segment (start 157 91.8) (end 157 90.35) (width 0.25) (layer F.Cu) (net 7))
 (segment (start 162.109413 98.6) (end 163.709413 97) (width 0.25) (layer F.Cu) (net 5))
 (segment (start 163.709413 97) (end 167.65 97) (width 0.25) (layer F.Cu) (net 5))
 (segment (start 160.05 98.6) (end 162.109413 98.6) (width 0.25) (layer F.Cu) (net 5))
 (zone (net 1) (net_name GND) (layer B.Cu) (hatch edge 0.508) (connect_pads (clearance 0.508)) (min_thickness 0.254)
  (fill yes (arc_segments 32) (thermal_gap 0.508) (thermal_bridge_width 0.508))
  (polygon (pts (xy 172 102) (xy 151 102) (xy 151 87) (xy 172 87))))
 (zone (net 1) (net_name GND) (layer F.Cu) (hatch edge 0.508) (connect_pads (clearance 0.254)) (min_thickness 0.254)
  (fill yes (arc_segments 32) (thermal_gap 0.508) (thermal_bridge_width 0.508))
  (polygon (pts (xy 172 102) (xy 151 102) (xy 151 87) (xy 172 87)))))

